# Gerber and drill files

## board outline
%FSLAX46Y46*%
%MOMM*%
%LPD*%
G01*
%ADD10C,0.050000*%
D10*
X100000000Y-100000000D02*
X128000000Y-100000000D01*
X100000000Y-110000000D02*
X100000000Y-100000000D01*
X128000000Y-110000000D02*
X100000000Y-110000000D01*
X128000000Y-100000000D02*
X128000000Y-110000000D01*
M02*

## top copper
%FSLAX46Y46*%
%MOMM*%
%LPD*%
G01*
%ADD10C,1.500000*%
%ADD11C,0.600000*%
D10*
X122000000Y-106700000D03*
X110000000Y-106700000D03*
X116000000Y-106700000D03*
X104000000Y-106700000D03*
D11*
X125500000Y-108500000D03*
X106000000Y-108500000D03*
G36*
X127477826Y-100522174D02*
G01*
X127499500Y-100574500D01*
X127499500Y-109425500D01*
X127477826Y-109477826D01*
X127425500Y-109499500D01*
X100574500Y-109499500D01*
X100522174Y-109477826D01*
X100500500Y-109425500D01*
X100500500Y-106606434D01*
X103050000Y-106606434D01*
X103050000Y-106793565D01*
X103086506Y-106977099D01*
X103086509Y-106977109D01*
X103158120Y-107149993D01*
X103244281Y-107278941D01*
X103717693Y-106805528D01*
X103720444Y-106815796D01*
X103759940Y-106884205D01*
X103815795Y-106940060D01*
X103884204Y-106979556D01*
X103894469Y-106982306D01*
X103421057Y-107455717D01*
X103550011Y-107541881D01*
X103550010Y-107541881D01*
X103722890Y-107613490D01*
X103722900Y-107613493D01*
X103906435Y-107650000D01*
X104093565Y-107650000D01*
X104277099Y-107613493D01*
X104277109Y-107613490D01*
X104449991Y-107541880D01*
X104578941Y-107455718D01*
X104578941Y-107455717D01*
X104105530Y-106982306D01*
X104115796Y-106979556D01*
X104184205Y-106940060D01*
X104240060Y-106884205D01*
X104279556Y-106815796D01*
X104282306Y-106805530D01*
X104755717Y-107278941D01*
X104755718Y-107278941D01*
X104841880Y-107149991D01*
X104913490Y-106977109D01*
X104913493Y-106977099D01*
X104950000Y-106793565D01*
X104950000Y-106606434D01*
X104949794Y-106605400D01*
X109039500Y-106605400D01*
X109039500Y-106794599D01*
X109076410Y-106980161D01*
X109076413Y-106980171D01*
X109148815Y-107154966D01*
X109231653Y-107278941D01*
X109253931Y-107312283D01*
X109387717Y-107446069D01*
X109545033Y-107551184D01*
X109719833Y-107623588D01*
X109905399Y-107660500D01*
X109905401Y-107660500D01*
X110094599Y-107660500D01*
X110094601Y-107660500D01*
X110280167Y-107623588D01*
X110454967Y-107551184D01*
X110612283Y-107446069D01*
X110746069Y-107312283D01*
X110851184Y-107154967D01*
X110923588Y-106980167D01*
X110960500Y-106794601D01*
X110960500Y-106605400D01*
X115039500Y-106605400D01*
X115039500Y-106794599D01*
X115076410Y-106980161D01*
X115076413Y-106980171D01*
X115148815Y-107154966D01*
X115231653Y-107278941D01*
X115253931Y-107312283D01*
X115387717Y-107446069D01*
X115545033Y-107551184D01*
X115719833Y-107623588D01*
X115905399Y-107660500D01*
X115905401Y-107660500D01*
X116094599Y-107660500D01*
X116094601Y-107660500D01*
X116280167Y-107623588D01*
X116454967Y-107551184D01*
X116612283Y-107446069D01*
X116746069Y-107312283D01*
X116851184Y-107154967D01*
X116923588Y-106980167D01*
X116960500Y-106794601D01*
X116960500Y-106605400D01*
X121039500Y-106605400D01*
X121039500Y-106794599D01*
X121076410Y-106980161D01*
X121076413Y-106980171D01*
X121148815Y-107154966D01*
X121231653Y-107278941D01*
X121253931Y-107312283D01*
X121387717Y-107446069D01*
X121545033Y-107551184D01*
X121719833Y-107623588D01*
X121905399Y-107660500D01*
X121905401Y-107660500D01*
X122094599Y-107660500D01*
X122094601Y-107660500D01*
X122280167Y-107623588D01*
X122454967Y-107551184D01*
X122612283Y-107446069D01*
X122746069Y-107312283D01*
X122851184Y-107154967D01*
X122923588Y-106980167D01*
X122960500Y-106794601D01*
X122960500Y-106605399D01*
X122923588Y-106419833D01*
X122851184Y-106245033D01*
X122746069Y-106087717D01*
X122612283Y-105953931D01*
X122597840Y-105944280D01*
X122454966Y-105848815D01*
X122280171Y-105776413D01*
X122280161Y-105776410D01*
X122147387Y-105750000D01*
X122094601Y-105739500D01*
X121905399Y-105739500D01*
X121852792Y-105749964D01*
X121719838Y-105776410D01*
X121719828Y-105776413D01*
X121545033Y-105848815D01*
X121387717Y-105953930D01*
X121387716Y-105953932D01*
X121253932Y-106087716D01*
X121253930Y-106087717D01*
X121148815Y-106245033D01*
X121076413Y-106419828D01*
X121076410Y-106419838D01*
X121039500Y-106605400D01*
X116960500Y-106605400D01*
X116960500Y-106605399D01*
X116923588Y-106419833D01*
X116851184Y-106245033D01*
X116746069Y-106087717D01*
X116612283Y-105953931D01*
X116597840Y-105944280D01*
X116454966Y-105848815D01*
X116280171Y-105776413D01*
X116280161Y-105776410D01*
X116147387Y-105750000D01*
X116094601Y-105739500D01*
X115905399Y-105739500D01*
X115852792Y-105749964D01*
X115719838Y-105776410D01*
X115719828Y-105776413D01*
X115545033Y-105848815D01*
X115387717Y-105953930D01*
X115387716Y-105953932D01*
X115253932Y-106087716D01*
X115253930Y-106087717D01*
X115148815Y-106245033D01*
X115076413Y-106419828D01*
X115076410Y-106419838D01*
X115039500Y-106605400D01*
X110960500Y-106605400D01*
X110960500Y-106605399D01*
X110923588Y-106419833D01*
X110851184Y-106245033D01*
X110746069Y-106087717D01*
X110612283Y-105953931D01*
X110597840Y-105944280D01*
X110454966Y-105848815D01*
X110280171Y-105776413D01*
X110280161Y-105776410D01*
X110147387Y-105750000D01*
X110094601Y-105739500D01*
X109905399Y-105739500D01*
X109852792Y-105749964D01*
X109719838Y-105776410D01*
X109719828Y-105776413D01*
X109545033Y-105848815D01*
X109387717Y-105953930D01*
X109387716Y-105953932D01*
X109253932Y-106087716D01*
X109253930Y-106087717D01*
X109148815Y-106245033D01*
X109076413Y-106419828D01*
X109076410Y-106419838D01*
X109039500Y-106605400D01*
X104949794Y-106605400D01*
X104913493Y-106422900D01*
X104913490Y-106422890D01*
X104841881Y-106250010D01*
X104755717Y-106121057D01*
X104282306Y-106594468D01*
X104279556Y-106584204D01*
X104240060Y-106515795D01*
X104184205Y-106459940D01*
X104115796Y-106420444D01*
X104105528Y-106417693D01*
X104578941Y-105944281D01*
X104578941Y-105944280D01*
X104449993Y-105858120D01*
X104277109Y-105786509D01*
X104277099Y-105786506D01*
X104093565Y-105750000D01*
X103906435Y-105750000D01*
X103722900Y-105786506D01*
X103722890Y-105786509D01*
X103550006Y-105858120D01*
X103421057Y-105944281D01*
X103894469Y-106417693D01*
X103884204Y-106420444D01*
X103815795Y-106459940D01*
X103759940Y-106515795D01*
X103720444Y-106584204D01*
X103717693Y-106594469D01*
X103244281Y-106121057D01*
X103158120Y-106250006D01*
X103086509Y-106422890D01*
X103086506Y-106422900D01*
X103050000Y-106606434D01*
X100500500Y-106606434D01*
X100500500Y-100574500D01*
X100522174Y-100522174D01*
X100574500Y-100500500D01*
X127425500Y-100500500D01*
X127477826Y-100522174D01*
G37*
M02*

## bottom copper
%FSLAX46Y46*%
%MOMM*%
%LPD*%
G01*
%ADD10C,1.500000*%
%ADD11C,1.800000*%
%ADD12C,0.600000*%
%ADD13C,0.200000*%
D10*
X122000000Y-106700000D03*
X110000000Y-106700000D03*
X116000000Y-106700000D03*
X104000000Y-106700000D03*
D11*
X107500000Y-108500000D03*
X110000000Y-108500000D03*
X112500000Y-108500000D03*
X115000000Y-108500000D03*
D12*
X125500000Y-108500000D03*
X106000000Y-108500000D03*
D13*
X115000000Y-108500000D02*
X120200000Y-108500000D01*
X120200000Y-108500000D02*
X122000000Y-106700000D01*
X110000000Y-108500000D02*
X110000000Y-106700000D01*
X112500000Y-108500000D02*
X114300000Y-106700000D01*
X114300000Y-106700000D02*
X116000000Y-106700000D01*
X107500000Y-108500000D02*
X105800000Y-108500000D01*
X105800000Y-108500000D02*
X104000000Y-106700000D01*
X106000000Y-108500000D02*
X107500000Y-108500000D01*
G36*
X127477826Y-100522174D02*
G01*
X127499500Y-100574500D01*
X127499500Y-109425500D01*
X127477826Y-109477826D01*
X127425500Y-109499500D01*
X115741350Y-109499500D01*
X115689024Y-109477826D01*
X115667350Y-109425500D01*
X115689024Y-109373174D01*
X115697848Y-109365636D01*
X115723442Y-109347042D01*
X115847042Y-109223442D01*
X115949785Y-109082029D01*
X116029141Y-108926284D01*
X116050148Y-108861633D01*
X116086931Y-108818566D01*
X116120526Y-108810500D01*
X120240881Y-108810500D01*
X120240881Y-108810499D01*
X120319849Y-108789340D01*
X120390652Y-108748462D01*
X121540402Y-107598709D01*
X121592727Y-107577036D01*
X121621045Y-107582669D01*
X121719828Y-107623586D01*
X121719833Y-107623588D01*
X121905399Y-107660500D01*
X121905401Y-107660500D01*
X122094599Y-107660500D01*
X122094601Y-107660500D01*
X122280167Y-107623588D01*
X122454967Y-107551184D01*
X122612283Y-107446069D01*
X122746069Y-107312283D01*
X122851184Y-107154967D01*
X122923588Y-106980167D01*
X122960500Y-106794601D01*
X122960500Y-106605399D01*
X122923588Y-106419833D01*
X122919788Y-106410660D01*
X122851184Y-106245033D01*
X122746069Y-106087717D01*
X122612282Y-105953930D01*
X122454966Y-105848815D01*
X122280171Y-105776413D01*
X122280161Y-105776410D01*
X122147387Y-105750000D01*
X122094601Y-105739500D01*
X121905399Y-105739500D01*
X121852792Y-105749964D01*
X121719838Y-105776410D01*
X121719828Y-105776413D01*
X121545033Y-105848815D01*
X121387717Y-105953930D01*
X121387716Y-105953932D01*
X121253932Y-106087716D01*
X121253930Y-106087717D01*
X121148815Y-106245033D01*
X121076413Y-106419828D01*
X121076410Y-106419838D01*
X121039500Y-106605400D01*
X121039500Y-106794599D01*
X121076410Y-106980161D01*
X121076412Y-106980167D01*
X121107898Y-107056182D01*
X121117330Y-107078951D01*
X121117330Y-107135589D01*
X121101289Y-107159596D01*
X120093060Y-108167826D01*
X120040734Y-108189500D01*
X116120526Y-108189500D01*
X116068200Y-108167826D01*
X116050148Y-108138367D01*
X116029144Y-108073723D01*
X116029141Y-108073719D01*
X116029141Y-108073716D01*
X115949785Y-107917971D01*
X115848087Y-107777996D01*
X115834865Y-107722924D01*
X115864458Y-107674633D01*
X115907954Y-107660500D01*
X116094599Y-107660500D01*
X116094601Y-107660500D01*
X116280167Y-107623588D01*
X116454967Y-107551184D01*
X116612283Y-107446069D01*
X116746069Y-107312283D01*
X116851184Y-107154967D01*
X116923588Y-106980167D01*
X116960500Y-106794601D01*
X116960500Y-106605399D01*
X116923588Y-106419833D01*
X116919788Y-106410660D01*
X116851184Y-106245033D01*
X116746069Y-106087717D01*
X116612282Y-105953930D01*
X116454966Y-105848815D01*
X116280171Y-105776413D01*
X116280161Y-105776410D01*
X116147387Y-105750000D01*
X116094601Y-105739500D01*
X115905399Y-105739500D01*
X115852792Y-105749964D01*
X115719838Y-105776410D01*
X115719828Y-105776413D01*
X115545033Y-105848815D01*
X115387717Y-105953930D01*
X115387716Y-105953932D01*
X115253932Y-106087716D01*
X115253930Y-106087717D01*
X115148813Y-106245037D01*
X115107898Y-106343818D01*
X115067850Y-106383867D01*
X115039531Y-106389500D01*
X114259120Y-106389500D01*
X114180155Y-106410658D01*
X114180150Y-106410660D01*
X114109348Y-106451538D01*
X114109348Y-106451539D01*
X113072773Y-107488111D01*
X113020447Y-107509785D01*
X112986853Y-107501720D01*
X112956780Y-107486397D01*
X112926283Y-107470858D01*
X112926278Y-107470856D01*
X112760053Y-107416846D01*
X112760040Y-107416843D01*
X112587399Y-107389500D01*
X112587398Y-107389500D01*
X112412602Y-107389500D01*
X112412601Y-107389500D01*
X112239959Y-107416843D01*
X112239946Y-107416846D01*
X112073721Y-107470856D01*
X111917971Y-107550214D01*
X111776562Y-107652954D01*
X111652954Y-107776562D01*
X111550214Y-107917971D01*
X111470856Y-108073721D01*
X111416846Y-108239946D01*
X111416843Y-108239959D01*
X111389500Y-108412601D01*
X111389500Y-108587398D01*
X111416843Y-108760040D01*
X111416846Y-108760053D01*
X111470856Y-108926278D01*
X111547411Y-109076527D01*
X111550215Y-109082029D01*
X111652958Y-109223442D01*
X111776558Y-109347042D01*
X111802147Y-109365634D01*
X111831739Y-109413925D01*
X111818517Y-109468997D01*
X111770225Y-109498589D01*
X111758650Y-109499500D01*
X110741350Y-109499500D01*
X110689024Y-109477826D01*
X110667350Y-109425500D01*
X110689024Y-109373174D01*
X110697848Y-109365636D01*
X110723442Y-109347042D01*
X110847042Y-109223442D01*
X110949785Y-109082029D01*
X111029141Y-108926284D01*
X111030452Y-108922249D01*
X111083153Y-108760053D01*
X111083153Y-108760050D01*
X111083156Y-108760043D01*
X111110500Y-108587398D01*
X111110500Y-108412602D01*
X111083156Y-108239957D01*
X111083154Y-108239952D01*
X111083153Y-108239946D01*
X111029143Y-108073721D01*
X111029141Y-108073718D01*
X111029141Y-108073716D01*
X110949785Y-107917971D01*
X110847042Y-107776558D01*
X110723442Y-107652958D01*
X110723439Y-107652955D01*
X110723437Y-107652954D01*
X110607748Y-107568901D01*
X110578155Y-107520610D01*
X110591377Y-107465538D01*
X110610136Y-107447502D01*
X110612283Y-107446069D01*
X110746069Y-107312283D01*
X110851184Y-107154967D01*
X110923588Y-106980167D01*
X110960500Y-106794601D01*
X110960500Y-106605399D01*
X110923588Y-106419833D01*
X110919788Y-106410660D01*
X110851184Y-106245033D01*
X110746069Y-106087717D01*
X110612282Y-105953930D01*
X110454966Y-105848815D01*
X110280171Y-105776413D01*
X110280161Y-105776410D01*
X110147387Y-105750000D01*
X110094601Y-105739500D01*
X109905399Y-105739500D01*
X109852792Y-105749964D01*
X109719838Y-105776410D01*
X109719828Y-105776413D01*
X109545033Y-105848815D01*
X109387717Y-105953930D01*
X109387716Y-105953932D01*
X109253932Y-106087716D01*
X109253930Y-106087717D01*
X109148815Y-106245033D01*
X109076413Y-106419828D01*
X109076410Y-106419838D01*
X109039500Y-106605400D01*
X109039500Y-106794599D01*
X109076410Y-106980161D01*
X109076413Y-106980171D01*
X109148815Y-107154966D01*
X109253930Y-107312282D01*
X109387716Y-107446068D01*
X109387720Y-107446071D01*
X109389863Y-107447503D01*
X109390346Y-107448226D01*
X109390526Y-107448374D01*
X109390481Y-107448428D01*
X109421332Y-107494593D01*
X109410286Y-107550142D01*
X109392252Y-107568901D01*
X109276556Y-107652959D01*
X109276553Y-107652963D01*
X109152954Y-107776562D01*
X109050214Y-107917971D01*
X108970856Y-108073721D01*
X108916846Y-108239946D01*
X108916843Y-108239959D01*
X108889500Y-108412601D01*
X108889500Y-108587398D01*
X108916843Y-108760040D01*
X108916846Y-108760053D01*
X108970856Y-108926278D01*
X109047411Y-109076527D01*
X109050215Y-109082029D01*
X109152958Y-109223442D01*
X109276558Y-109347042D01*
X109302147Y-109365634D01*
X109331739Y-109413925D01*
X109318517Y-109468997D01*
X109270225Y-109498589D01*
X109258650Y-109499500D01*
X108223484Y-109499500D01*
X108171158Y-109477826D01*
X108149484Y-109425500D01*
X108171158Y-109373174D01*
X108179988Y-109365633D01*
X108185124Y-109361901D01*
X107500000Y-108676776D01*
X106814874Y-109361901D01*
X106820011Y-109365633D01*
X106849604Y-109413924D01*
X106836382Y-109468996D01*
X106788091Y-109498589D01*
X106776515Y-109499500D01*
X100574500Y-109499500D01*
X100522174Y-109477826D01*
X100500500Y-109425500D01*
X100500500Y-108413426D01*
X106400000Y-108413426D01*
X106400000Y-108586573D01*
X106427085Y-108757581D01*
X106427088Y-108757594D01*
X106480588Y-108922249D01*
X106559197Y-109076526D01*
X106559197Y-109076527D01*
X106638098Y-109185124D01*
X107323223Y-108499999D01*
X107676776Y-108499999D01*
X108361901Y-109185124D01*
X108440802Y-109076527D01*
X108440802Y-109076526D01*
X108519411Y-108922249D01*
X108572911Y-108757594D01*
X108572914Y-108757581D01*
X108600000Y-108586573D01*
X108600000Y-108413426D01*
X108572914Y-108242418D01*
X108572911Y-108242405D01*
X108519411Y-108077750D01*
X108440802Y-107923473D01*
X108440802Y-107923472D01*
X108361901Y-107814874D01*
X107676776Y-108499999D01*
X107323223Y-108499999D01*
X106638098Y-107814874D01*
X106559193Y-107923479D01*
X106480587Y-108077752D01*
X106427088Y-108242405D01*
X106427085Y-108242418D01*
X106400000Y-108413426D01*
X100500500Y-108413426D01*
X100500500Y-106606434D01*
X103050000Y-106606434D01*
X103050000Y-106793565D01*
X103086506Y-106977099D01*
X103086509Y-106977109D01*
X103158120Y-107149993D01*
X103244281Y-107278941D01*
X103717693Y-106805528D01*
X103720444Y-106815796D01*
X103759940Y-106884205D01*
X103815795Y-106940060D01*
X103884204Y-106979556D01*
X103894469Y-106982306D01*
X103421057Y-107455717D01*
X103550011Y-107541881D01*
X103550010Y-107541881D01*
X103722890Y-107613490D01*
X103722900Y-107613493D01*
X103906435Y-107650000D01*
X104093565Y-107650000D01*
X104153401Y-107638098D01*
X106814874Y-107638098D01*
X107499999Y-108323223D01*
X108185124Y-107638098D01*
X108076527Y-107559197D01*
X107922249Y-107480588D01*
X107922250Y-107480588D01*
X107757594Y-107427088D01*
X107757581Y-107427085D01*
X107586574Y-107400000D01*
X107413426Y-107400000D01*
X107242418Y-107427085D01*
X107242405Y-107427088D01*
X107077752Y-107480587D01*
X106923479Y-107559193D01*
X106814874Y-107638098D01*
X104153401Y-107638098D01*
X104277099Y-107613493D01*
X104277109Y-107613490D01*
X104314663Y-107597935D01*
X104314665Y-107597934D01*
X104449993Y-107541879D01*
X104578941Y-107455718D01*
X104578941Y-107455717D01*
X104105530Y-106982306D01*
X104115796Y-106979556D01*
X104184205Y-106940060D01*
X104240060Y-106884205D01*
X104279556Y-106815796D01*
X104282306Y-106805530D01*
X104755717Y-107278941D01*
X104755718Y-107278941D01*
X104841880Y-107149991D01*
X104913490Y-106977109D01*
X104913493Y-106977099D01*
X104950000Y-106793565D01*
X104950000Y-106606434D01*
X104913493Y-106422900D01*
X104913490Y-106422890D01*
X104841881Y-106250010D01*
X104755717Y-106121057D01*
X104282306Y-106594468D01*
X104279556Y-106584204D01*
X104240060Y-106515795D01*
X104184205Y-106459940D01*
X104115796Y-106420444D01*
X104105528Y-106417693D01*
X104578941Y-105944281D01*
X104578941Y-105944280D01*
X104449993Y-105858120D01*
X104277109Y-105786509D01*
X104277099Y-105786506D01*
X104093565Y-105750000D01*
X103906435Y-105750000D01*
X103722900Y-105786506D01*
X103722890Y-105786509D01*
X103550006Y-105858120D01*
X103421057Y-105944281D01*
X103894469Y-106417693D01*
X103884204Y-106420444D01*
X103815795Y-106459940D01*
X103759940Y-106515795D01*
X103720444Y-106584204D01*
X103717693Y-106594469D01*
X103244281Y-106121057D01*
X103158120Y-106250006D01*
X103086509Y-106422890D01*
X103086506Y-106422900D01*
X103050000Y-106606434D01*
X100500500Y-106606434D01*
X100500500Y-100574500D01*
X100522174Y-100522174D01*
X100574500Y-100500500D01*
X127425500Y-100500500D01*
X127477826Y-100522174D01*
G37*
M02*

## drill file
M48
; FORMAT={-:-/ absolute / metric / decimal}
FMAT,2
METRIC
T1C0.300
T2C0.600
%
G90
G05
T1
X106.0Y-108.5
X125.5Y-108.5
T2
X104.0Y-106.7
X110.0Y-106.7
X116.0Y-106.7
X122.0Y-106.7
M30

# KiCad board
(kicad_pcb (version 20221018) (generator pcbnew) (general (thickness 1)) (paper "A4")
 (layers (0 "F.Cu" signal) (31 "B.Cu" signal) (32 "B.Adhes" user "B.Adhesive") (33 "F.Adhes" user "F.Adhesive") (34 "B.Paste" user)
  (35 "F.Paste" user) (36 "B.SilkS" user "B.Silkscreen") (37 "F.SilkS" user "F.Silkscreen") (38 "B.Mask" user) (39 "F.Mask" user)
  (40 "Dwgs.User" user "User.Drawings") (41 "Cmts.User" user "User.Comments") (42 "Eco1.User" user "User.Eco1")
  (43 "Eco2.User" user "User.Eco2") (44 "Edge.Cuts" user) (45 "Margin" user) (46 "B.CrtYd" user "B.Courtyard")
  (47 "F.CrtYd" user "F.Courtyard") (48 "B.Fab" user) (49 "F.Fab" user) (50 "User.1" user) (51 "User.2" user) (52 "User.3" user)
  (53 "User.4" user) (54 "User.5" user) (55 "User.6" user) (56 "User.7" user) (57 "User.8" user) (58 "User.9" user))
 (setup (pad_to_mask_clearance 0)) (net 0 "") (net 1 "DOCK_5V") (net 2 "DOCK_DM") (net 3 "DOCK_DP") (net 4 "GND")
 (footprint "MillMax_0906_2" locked (layer "F.Cu") (at 122 106.7)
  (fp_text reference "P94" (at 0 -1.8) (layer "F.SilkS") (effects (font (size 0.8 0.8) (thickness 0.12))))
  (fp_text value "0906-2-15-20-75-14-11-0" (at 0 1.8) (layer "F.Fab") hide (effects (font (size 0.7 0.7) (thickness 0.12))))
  (pad "1" thru_hole circle locked (at 0 0) (size 1.5 1.5) (drill 0.6) (layers "*.Cu" "*.Mask") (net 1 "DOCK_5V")))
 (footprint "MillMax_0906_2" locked (layer "F.Cu") (at 110 106.7)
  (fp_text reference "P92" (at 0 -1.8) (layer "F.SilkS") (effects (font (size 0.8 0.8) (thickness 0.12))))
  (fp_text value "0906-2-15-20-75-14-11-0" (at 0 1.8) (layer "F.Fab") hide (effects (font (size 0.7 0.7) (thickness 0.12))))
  (pad "1" thru_hole circle locked (at 0 0) (size 1.5 1.5) (drill 0.6) (layers "*.Cu" "*.Mask") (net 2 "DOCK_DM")))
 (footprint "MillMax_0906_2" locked (layer "F.Cu") (at 116 106.7)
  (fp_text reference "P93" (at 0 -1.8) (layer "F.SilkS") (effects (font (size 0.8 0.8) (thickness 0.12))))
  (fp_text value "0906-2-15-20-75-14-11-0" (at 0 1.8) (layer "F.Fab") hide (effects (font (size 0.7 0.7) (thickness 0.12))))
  (pad "1" thru_hole circle locked (at 0 0) (size 1.5 1.5) (drill 0.6) (layers "*.Cu" "*.Mask") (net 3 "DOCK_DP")))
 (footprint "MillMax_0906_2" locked (layer "F.Cu") (at 104 106.7)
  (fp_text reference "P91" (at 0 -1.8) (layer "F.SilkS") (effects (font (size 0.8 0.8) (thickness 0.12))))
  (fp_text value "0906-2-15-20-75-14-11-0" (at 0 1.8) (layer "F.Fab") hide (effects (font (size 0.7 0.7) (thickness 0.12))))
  (pad "1" thru_hole circle locked (at 0 0) (size 1.5 1.5) (drill 0.6) (layers "*.Cu" "*.Mask") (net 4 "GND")))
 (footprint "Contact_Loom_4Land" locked (layer "B.Cu") (at 107.5 108.5)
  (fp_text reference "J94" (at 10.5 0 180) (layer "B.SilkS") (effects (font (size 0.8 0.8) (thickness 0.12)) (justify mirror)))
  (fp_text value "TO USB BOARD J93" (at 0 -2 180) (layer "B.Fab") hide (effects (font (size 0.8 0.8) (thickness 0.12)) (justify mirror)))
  (pad "1" smd circle locked (at 0 0) (size 1.8 1.8) (layers "B.Cu" "B.Paste" "B.Mask") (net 4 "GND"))
  (pad "2" smd circle locked (at 2.5 0) (size 1.8 1.8) (layers "B.Cu" "B.Paste" "B.Mask") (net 2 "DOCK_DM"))
  (pad "3" smd circle locked (at 5 0) (size 1.8 1.8) (layers "B.Cu" "B.Paste" "B.Mask") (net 3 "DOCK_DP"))
  (pad "4" smd circle locked (at 7.5 0) (size 1.8 1.8) (layers "B.Cu" "B.Paste" "B.Mask") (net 1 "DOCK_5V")))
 (gr_line (start 100 100) (end 128 100) (stroke (width 0.05) (type default)) (layer "Edge.Cuts"))
 (gr_line (start 100 110) (end 100 100) (stroke (width 0.05) (type default)) (layer "Edge.Cuts"))
 (gr_line (start 128 110) (end 100 110) (stroke (width 0.05) (type default)) (layer "Edge.Cuts"))
 (gr_line (start 128 100) (end 128 110) (stroke (width 0.05) (type default)) (layer "Edge.Cuts"))
 (segment (start 115 108.5) (end 120.2 108.5) (width 0.2) (layer "B.Cu") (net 1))
 (segment (start 120.2 108.5) (end 122 106.7) (width 0.2) (layer "B.Cu") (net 1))
 (segment (start 110 108.5) (end 110 106.7) (width 0.2) (layer "B.Cu") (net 2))
 (segment (start 112.5 108.5) (end 114.3 106.7) (width 0.2) (layer "B.Cu") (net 3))
 (segment (start 114.3 106.7) (end 116 106.7) (width 0.2) (layer "B.Cu") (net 3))
 (via (at 125.5 108.5) (size 0.6) (drill 0.3) (layers "F.Cu" "B.Cu") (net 4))
 (via (at 106 108.5) (size 0.6) (drill 0.3) (layers "F.Cu" "B.Cu") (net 4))
 (segment (start 107.5 108.5) (end 105.8 108.5) (width 0.2) (layer "B.Cu") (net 4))
 (segment (start 105.8 108.5) (end 104 106.7) (width 0.2) (layer "B.Cu") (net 4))
 (segment (start 106 108.5) (end 107.5 108.5) (width 0.2) (layer "B.Cu") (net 4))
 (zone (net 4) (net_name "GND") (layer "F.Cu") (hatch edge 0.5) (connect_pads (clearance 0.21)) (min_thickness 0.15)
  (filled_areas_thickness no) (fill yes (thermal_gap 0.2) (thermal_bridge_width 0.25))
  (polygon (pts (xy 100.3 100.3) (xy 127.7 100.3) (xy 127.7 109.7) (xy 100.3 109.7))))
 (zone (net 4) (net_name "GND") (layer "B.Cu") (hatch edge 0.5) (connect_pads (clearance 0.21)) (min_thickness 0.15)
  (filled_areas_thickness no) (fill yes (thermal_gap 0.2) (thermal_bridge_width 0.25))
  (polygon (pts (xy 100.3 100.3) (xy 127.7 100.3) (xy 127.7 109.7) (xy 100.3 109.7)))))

